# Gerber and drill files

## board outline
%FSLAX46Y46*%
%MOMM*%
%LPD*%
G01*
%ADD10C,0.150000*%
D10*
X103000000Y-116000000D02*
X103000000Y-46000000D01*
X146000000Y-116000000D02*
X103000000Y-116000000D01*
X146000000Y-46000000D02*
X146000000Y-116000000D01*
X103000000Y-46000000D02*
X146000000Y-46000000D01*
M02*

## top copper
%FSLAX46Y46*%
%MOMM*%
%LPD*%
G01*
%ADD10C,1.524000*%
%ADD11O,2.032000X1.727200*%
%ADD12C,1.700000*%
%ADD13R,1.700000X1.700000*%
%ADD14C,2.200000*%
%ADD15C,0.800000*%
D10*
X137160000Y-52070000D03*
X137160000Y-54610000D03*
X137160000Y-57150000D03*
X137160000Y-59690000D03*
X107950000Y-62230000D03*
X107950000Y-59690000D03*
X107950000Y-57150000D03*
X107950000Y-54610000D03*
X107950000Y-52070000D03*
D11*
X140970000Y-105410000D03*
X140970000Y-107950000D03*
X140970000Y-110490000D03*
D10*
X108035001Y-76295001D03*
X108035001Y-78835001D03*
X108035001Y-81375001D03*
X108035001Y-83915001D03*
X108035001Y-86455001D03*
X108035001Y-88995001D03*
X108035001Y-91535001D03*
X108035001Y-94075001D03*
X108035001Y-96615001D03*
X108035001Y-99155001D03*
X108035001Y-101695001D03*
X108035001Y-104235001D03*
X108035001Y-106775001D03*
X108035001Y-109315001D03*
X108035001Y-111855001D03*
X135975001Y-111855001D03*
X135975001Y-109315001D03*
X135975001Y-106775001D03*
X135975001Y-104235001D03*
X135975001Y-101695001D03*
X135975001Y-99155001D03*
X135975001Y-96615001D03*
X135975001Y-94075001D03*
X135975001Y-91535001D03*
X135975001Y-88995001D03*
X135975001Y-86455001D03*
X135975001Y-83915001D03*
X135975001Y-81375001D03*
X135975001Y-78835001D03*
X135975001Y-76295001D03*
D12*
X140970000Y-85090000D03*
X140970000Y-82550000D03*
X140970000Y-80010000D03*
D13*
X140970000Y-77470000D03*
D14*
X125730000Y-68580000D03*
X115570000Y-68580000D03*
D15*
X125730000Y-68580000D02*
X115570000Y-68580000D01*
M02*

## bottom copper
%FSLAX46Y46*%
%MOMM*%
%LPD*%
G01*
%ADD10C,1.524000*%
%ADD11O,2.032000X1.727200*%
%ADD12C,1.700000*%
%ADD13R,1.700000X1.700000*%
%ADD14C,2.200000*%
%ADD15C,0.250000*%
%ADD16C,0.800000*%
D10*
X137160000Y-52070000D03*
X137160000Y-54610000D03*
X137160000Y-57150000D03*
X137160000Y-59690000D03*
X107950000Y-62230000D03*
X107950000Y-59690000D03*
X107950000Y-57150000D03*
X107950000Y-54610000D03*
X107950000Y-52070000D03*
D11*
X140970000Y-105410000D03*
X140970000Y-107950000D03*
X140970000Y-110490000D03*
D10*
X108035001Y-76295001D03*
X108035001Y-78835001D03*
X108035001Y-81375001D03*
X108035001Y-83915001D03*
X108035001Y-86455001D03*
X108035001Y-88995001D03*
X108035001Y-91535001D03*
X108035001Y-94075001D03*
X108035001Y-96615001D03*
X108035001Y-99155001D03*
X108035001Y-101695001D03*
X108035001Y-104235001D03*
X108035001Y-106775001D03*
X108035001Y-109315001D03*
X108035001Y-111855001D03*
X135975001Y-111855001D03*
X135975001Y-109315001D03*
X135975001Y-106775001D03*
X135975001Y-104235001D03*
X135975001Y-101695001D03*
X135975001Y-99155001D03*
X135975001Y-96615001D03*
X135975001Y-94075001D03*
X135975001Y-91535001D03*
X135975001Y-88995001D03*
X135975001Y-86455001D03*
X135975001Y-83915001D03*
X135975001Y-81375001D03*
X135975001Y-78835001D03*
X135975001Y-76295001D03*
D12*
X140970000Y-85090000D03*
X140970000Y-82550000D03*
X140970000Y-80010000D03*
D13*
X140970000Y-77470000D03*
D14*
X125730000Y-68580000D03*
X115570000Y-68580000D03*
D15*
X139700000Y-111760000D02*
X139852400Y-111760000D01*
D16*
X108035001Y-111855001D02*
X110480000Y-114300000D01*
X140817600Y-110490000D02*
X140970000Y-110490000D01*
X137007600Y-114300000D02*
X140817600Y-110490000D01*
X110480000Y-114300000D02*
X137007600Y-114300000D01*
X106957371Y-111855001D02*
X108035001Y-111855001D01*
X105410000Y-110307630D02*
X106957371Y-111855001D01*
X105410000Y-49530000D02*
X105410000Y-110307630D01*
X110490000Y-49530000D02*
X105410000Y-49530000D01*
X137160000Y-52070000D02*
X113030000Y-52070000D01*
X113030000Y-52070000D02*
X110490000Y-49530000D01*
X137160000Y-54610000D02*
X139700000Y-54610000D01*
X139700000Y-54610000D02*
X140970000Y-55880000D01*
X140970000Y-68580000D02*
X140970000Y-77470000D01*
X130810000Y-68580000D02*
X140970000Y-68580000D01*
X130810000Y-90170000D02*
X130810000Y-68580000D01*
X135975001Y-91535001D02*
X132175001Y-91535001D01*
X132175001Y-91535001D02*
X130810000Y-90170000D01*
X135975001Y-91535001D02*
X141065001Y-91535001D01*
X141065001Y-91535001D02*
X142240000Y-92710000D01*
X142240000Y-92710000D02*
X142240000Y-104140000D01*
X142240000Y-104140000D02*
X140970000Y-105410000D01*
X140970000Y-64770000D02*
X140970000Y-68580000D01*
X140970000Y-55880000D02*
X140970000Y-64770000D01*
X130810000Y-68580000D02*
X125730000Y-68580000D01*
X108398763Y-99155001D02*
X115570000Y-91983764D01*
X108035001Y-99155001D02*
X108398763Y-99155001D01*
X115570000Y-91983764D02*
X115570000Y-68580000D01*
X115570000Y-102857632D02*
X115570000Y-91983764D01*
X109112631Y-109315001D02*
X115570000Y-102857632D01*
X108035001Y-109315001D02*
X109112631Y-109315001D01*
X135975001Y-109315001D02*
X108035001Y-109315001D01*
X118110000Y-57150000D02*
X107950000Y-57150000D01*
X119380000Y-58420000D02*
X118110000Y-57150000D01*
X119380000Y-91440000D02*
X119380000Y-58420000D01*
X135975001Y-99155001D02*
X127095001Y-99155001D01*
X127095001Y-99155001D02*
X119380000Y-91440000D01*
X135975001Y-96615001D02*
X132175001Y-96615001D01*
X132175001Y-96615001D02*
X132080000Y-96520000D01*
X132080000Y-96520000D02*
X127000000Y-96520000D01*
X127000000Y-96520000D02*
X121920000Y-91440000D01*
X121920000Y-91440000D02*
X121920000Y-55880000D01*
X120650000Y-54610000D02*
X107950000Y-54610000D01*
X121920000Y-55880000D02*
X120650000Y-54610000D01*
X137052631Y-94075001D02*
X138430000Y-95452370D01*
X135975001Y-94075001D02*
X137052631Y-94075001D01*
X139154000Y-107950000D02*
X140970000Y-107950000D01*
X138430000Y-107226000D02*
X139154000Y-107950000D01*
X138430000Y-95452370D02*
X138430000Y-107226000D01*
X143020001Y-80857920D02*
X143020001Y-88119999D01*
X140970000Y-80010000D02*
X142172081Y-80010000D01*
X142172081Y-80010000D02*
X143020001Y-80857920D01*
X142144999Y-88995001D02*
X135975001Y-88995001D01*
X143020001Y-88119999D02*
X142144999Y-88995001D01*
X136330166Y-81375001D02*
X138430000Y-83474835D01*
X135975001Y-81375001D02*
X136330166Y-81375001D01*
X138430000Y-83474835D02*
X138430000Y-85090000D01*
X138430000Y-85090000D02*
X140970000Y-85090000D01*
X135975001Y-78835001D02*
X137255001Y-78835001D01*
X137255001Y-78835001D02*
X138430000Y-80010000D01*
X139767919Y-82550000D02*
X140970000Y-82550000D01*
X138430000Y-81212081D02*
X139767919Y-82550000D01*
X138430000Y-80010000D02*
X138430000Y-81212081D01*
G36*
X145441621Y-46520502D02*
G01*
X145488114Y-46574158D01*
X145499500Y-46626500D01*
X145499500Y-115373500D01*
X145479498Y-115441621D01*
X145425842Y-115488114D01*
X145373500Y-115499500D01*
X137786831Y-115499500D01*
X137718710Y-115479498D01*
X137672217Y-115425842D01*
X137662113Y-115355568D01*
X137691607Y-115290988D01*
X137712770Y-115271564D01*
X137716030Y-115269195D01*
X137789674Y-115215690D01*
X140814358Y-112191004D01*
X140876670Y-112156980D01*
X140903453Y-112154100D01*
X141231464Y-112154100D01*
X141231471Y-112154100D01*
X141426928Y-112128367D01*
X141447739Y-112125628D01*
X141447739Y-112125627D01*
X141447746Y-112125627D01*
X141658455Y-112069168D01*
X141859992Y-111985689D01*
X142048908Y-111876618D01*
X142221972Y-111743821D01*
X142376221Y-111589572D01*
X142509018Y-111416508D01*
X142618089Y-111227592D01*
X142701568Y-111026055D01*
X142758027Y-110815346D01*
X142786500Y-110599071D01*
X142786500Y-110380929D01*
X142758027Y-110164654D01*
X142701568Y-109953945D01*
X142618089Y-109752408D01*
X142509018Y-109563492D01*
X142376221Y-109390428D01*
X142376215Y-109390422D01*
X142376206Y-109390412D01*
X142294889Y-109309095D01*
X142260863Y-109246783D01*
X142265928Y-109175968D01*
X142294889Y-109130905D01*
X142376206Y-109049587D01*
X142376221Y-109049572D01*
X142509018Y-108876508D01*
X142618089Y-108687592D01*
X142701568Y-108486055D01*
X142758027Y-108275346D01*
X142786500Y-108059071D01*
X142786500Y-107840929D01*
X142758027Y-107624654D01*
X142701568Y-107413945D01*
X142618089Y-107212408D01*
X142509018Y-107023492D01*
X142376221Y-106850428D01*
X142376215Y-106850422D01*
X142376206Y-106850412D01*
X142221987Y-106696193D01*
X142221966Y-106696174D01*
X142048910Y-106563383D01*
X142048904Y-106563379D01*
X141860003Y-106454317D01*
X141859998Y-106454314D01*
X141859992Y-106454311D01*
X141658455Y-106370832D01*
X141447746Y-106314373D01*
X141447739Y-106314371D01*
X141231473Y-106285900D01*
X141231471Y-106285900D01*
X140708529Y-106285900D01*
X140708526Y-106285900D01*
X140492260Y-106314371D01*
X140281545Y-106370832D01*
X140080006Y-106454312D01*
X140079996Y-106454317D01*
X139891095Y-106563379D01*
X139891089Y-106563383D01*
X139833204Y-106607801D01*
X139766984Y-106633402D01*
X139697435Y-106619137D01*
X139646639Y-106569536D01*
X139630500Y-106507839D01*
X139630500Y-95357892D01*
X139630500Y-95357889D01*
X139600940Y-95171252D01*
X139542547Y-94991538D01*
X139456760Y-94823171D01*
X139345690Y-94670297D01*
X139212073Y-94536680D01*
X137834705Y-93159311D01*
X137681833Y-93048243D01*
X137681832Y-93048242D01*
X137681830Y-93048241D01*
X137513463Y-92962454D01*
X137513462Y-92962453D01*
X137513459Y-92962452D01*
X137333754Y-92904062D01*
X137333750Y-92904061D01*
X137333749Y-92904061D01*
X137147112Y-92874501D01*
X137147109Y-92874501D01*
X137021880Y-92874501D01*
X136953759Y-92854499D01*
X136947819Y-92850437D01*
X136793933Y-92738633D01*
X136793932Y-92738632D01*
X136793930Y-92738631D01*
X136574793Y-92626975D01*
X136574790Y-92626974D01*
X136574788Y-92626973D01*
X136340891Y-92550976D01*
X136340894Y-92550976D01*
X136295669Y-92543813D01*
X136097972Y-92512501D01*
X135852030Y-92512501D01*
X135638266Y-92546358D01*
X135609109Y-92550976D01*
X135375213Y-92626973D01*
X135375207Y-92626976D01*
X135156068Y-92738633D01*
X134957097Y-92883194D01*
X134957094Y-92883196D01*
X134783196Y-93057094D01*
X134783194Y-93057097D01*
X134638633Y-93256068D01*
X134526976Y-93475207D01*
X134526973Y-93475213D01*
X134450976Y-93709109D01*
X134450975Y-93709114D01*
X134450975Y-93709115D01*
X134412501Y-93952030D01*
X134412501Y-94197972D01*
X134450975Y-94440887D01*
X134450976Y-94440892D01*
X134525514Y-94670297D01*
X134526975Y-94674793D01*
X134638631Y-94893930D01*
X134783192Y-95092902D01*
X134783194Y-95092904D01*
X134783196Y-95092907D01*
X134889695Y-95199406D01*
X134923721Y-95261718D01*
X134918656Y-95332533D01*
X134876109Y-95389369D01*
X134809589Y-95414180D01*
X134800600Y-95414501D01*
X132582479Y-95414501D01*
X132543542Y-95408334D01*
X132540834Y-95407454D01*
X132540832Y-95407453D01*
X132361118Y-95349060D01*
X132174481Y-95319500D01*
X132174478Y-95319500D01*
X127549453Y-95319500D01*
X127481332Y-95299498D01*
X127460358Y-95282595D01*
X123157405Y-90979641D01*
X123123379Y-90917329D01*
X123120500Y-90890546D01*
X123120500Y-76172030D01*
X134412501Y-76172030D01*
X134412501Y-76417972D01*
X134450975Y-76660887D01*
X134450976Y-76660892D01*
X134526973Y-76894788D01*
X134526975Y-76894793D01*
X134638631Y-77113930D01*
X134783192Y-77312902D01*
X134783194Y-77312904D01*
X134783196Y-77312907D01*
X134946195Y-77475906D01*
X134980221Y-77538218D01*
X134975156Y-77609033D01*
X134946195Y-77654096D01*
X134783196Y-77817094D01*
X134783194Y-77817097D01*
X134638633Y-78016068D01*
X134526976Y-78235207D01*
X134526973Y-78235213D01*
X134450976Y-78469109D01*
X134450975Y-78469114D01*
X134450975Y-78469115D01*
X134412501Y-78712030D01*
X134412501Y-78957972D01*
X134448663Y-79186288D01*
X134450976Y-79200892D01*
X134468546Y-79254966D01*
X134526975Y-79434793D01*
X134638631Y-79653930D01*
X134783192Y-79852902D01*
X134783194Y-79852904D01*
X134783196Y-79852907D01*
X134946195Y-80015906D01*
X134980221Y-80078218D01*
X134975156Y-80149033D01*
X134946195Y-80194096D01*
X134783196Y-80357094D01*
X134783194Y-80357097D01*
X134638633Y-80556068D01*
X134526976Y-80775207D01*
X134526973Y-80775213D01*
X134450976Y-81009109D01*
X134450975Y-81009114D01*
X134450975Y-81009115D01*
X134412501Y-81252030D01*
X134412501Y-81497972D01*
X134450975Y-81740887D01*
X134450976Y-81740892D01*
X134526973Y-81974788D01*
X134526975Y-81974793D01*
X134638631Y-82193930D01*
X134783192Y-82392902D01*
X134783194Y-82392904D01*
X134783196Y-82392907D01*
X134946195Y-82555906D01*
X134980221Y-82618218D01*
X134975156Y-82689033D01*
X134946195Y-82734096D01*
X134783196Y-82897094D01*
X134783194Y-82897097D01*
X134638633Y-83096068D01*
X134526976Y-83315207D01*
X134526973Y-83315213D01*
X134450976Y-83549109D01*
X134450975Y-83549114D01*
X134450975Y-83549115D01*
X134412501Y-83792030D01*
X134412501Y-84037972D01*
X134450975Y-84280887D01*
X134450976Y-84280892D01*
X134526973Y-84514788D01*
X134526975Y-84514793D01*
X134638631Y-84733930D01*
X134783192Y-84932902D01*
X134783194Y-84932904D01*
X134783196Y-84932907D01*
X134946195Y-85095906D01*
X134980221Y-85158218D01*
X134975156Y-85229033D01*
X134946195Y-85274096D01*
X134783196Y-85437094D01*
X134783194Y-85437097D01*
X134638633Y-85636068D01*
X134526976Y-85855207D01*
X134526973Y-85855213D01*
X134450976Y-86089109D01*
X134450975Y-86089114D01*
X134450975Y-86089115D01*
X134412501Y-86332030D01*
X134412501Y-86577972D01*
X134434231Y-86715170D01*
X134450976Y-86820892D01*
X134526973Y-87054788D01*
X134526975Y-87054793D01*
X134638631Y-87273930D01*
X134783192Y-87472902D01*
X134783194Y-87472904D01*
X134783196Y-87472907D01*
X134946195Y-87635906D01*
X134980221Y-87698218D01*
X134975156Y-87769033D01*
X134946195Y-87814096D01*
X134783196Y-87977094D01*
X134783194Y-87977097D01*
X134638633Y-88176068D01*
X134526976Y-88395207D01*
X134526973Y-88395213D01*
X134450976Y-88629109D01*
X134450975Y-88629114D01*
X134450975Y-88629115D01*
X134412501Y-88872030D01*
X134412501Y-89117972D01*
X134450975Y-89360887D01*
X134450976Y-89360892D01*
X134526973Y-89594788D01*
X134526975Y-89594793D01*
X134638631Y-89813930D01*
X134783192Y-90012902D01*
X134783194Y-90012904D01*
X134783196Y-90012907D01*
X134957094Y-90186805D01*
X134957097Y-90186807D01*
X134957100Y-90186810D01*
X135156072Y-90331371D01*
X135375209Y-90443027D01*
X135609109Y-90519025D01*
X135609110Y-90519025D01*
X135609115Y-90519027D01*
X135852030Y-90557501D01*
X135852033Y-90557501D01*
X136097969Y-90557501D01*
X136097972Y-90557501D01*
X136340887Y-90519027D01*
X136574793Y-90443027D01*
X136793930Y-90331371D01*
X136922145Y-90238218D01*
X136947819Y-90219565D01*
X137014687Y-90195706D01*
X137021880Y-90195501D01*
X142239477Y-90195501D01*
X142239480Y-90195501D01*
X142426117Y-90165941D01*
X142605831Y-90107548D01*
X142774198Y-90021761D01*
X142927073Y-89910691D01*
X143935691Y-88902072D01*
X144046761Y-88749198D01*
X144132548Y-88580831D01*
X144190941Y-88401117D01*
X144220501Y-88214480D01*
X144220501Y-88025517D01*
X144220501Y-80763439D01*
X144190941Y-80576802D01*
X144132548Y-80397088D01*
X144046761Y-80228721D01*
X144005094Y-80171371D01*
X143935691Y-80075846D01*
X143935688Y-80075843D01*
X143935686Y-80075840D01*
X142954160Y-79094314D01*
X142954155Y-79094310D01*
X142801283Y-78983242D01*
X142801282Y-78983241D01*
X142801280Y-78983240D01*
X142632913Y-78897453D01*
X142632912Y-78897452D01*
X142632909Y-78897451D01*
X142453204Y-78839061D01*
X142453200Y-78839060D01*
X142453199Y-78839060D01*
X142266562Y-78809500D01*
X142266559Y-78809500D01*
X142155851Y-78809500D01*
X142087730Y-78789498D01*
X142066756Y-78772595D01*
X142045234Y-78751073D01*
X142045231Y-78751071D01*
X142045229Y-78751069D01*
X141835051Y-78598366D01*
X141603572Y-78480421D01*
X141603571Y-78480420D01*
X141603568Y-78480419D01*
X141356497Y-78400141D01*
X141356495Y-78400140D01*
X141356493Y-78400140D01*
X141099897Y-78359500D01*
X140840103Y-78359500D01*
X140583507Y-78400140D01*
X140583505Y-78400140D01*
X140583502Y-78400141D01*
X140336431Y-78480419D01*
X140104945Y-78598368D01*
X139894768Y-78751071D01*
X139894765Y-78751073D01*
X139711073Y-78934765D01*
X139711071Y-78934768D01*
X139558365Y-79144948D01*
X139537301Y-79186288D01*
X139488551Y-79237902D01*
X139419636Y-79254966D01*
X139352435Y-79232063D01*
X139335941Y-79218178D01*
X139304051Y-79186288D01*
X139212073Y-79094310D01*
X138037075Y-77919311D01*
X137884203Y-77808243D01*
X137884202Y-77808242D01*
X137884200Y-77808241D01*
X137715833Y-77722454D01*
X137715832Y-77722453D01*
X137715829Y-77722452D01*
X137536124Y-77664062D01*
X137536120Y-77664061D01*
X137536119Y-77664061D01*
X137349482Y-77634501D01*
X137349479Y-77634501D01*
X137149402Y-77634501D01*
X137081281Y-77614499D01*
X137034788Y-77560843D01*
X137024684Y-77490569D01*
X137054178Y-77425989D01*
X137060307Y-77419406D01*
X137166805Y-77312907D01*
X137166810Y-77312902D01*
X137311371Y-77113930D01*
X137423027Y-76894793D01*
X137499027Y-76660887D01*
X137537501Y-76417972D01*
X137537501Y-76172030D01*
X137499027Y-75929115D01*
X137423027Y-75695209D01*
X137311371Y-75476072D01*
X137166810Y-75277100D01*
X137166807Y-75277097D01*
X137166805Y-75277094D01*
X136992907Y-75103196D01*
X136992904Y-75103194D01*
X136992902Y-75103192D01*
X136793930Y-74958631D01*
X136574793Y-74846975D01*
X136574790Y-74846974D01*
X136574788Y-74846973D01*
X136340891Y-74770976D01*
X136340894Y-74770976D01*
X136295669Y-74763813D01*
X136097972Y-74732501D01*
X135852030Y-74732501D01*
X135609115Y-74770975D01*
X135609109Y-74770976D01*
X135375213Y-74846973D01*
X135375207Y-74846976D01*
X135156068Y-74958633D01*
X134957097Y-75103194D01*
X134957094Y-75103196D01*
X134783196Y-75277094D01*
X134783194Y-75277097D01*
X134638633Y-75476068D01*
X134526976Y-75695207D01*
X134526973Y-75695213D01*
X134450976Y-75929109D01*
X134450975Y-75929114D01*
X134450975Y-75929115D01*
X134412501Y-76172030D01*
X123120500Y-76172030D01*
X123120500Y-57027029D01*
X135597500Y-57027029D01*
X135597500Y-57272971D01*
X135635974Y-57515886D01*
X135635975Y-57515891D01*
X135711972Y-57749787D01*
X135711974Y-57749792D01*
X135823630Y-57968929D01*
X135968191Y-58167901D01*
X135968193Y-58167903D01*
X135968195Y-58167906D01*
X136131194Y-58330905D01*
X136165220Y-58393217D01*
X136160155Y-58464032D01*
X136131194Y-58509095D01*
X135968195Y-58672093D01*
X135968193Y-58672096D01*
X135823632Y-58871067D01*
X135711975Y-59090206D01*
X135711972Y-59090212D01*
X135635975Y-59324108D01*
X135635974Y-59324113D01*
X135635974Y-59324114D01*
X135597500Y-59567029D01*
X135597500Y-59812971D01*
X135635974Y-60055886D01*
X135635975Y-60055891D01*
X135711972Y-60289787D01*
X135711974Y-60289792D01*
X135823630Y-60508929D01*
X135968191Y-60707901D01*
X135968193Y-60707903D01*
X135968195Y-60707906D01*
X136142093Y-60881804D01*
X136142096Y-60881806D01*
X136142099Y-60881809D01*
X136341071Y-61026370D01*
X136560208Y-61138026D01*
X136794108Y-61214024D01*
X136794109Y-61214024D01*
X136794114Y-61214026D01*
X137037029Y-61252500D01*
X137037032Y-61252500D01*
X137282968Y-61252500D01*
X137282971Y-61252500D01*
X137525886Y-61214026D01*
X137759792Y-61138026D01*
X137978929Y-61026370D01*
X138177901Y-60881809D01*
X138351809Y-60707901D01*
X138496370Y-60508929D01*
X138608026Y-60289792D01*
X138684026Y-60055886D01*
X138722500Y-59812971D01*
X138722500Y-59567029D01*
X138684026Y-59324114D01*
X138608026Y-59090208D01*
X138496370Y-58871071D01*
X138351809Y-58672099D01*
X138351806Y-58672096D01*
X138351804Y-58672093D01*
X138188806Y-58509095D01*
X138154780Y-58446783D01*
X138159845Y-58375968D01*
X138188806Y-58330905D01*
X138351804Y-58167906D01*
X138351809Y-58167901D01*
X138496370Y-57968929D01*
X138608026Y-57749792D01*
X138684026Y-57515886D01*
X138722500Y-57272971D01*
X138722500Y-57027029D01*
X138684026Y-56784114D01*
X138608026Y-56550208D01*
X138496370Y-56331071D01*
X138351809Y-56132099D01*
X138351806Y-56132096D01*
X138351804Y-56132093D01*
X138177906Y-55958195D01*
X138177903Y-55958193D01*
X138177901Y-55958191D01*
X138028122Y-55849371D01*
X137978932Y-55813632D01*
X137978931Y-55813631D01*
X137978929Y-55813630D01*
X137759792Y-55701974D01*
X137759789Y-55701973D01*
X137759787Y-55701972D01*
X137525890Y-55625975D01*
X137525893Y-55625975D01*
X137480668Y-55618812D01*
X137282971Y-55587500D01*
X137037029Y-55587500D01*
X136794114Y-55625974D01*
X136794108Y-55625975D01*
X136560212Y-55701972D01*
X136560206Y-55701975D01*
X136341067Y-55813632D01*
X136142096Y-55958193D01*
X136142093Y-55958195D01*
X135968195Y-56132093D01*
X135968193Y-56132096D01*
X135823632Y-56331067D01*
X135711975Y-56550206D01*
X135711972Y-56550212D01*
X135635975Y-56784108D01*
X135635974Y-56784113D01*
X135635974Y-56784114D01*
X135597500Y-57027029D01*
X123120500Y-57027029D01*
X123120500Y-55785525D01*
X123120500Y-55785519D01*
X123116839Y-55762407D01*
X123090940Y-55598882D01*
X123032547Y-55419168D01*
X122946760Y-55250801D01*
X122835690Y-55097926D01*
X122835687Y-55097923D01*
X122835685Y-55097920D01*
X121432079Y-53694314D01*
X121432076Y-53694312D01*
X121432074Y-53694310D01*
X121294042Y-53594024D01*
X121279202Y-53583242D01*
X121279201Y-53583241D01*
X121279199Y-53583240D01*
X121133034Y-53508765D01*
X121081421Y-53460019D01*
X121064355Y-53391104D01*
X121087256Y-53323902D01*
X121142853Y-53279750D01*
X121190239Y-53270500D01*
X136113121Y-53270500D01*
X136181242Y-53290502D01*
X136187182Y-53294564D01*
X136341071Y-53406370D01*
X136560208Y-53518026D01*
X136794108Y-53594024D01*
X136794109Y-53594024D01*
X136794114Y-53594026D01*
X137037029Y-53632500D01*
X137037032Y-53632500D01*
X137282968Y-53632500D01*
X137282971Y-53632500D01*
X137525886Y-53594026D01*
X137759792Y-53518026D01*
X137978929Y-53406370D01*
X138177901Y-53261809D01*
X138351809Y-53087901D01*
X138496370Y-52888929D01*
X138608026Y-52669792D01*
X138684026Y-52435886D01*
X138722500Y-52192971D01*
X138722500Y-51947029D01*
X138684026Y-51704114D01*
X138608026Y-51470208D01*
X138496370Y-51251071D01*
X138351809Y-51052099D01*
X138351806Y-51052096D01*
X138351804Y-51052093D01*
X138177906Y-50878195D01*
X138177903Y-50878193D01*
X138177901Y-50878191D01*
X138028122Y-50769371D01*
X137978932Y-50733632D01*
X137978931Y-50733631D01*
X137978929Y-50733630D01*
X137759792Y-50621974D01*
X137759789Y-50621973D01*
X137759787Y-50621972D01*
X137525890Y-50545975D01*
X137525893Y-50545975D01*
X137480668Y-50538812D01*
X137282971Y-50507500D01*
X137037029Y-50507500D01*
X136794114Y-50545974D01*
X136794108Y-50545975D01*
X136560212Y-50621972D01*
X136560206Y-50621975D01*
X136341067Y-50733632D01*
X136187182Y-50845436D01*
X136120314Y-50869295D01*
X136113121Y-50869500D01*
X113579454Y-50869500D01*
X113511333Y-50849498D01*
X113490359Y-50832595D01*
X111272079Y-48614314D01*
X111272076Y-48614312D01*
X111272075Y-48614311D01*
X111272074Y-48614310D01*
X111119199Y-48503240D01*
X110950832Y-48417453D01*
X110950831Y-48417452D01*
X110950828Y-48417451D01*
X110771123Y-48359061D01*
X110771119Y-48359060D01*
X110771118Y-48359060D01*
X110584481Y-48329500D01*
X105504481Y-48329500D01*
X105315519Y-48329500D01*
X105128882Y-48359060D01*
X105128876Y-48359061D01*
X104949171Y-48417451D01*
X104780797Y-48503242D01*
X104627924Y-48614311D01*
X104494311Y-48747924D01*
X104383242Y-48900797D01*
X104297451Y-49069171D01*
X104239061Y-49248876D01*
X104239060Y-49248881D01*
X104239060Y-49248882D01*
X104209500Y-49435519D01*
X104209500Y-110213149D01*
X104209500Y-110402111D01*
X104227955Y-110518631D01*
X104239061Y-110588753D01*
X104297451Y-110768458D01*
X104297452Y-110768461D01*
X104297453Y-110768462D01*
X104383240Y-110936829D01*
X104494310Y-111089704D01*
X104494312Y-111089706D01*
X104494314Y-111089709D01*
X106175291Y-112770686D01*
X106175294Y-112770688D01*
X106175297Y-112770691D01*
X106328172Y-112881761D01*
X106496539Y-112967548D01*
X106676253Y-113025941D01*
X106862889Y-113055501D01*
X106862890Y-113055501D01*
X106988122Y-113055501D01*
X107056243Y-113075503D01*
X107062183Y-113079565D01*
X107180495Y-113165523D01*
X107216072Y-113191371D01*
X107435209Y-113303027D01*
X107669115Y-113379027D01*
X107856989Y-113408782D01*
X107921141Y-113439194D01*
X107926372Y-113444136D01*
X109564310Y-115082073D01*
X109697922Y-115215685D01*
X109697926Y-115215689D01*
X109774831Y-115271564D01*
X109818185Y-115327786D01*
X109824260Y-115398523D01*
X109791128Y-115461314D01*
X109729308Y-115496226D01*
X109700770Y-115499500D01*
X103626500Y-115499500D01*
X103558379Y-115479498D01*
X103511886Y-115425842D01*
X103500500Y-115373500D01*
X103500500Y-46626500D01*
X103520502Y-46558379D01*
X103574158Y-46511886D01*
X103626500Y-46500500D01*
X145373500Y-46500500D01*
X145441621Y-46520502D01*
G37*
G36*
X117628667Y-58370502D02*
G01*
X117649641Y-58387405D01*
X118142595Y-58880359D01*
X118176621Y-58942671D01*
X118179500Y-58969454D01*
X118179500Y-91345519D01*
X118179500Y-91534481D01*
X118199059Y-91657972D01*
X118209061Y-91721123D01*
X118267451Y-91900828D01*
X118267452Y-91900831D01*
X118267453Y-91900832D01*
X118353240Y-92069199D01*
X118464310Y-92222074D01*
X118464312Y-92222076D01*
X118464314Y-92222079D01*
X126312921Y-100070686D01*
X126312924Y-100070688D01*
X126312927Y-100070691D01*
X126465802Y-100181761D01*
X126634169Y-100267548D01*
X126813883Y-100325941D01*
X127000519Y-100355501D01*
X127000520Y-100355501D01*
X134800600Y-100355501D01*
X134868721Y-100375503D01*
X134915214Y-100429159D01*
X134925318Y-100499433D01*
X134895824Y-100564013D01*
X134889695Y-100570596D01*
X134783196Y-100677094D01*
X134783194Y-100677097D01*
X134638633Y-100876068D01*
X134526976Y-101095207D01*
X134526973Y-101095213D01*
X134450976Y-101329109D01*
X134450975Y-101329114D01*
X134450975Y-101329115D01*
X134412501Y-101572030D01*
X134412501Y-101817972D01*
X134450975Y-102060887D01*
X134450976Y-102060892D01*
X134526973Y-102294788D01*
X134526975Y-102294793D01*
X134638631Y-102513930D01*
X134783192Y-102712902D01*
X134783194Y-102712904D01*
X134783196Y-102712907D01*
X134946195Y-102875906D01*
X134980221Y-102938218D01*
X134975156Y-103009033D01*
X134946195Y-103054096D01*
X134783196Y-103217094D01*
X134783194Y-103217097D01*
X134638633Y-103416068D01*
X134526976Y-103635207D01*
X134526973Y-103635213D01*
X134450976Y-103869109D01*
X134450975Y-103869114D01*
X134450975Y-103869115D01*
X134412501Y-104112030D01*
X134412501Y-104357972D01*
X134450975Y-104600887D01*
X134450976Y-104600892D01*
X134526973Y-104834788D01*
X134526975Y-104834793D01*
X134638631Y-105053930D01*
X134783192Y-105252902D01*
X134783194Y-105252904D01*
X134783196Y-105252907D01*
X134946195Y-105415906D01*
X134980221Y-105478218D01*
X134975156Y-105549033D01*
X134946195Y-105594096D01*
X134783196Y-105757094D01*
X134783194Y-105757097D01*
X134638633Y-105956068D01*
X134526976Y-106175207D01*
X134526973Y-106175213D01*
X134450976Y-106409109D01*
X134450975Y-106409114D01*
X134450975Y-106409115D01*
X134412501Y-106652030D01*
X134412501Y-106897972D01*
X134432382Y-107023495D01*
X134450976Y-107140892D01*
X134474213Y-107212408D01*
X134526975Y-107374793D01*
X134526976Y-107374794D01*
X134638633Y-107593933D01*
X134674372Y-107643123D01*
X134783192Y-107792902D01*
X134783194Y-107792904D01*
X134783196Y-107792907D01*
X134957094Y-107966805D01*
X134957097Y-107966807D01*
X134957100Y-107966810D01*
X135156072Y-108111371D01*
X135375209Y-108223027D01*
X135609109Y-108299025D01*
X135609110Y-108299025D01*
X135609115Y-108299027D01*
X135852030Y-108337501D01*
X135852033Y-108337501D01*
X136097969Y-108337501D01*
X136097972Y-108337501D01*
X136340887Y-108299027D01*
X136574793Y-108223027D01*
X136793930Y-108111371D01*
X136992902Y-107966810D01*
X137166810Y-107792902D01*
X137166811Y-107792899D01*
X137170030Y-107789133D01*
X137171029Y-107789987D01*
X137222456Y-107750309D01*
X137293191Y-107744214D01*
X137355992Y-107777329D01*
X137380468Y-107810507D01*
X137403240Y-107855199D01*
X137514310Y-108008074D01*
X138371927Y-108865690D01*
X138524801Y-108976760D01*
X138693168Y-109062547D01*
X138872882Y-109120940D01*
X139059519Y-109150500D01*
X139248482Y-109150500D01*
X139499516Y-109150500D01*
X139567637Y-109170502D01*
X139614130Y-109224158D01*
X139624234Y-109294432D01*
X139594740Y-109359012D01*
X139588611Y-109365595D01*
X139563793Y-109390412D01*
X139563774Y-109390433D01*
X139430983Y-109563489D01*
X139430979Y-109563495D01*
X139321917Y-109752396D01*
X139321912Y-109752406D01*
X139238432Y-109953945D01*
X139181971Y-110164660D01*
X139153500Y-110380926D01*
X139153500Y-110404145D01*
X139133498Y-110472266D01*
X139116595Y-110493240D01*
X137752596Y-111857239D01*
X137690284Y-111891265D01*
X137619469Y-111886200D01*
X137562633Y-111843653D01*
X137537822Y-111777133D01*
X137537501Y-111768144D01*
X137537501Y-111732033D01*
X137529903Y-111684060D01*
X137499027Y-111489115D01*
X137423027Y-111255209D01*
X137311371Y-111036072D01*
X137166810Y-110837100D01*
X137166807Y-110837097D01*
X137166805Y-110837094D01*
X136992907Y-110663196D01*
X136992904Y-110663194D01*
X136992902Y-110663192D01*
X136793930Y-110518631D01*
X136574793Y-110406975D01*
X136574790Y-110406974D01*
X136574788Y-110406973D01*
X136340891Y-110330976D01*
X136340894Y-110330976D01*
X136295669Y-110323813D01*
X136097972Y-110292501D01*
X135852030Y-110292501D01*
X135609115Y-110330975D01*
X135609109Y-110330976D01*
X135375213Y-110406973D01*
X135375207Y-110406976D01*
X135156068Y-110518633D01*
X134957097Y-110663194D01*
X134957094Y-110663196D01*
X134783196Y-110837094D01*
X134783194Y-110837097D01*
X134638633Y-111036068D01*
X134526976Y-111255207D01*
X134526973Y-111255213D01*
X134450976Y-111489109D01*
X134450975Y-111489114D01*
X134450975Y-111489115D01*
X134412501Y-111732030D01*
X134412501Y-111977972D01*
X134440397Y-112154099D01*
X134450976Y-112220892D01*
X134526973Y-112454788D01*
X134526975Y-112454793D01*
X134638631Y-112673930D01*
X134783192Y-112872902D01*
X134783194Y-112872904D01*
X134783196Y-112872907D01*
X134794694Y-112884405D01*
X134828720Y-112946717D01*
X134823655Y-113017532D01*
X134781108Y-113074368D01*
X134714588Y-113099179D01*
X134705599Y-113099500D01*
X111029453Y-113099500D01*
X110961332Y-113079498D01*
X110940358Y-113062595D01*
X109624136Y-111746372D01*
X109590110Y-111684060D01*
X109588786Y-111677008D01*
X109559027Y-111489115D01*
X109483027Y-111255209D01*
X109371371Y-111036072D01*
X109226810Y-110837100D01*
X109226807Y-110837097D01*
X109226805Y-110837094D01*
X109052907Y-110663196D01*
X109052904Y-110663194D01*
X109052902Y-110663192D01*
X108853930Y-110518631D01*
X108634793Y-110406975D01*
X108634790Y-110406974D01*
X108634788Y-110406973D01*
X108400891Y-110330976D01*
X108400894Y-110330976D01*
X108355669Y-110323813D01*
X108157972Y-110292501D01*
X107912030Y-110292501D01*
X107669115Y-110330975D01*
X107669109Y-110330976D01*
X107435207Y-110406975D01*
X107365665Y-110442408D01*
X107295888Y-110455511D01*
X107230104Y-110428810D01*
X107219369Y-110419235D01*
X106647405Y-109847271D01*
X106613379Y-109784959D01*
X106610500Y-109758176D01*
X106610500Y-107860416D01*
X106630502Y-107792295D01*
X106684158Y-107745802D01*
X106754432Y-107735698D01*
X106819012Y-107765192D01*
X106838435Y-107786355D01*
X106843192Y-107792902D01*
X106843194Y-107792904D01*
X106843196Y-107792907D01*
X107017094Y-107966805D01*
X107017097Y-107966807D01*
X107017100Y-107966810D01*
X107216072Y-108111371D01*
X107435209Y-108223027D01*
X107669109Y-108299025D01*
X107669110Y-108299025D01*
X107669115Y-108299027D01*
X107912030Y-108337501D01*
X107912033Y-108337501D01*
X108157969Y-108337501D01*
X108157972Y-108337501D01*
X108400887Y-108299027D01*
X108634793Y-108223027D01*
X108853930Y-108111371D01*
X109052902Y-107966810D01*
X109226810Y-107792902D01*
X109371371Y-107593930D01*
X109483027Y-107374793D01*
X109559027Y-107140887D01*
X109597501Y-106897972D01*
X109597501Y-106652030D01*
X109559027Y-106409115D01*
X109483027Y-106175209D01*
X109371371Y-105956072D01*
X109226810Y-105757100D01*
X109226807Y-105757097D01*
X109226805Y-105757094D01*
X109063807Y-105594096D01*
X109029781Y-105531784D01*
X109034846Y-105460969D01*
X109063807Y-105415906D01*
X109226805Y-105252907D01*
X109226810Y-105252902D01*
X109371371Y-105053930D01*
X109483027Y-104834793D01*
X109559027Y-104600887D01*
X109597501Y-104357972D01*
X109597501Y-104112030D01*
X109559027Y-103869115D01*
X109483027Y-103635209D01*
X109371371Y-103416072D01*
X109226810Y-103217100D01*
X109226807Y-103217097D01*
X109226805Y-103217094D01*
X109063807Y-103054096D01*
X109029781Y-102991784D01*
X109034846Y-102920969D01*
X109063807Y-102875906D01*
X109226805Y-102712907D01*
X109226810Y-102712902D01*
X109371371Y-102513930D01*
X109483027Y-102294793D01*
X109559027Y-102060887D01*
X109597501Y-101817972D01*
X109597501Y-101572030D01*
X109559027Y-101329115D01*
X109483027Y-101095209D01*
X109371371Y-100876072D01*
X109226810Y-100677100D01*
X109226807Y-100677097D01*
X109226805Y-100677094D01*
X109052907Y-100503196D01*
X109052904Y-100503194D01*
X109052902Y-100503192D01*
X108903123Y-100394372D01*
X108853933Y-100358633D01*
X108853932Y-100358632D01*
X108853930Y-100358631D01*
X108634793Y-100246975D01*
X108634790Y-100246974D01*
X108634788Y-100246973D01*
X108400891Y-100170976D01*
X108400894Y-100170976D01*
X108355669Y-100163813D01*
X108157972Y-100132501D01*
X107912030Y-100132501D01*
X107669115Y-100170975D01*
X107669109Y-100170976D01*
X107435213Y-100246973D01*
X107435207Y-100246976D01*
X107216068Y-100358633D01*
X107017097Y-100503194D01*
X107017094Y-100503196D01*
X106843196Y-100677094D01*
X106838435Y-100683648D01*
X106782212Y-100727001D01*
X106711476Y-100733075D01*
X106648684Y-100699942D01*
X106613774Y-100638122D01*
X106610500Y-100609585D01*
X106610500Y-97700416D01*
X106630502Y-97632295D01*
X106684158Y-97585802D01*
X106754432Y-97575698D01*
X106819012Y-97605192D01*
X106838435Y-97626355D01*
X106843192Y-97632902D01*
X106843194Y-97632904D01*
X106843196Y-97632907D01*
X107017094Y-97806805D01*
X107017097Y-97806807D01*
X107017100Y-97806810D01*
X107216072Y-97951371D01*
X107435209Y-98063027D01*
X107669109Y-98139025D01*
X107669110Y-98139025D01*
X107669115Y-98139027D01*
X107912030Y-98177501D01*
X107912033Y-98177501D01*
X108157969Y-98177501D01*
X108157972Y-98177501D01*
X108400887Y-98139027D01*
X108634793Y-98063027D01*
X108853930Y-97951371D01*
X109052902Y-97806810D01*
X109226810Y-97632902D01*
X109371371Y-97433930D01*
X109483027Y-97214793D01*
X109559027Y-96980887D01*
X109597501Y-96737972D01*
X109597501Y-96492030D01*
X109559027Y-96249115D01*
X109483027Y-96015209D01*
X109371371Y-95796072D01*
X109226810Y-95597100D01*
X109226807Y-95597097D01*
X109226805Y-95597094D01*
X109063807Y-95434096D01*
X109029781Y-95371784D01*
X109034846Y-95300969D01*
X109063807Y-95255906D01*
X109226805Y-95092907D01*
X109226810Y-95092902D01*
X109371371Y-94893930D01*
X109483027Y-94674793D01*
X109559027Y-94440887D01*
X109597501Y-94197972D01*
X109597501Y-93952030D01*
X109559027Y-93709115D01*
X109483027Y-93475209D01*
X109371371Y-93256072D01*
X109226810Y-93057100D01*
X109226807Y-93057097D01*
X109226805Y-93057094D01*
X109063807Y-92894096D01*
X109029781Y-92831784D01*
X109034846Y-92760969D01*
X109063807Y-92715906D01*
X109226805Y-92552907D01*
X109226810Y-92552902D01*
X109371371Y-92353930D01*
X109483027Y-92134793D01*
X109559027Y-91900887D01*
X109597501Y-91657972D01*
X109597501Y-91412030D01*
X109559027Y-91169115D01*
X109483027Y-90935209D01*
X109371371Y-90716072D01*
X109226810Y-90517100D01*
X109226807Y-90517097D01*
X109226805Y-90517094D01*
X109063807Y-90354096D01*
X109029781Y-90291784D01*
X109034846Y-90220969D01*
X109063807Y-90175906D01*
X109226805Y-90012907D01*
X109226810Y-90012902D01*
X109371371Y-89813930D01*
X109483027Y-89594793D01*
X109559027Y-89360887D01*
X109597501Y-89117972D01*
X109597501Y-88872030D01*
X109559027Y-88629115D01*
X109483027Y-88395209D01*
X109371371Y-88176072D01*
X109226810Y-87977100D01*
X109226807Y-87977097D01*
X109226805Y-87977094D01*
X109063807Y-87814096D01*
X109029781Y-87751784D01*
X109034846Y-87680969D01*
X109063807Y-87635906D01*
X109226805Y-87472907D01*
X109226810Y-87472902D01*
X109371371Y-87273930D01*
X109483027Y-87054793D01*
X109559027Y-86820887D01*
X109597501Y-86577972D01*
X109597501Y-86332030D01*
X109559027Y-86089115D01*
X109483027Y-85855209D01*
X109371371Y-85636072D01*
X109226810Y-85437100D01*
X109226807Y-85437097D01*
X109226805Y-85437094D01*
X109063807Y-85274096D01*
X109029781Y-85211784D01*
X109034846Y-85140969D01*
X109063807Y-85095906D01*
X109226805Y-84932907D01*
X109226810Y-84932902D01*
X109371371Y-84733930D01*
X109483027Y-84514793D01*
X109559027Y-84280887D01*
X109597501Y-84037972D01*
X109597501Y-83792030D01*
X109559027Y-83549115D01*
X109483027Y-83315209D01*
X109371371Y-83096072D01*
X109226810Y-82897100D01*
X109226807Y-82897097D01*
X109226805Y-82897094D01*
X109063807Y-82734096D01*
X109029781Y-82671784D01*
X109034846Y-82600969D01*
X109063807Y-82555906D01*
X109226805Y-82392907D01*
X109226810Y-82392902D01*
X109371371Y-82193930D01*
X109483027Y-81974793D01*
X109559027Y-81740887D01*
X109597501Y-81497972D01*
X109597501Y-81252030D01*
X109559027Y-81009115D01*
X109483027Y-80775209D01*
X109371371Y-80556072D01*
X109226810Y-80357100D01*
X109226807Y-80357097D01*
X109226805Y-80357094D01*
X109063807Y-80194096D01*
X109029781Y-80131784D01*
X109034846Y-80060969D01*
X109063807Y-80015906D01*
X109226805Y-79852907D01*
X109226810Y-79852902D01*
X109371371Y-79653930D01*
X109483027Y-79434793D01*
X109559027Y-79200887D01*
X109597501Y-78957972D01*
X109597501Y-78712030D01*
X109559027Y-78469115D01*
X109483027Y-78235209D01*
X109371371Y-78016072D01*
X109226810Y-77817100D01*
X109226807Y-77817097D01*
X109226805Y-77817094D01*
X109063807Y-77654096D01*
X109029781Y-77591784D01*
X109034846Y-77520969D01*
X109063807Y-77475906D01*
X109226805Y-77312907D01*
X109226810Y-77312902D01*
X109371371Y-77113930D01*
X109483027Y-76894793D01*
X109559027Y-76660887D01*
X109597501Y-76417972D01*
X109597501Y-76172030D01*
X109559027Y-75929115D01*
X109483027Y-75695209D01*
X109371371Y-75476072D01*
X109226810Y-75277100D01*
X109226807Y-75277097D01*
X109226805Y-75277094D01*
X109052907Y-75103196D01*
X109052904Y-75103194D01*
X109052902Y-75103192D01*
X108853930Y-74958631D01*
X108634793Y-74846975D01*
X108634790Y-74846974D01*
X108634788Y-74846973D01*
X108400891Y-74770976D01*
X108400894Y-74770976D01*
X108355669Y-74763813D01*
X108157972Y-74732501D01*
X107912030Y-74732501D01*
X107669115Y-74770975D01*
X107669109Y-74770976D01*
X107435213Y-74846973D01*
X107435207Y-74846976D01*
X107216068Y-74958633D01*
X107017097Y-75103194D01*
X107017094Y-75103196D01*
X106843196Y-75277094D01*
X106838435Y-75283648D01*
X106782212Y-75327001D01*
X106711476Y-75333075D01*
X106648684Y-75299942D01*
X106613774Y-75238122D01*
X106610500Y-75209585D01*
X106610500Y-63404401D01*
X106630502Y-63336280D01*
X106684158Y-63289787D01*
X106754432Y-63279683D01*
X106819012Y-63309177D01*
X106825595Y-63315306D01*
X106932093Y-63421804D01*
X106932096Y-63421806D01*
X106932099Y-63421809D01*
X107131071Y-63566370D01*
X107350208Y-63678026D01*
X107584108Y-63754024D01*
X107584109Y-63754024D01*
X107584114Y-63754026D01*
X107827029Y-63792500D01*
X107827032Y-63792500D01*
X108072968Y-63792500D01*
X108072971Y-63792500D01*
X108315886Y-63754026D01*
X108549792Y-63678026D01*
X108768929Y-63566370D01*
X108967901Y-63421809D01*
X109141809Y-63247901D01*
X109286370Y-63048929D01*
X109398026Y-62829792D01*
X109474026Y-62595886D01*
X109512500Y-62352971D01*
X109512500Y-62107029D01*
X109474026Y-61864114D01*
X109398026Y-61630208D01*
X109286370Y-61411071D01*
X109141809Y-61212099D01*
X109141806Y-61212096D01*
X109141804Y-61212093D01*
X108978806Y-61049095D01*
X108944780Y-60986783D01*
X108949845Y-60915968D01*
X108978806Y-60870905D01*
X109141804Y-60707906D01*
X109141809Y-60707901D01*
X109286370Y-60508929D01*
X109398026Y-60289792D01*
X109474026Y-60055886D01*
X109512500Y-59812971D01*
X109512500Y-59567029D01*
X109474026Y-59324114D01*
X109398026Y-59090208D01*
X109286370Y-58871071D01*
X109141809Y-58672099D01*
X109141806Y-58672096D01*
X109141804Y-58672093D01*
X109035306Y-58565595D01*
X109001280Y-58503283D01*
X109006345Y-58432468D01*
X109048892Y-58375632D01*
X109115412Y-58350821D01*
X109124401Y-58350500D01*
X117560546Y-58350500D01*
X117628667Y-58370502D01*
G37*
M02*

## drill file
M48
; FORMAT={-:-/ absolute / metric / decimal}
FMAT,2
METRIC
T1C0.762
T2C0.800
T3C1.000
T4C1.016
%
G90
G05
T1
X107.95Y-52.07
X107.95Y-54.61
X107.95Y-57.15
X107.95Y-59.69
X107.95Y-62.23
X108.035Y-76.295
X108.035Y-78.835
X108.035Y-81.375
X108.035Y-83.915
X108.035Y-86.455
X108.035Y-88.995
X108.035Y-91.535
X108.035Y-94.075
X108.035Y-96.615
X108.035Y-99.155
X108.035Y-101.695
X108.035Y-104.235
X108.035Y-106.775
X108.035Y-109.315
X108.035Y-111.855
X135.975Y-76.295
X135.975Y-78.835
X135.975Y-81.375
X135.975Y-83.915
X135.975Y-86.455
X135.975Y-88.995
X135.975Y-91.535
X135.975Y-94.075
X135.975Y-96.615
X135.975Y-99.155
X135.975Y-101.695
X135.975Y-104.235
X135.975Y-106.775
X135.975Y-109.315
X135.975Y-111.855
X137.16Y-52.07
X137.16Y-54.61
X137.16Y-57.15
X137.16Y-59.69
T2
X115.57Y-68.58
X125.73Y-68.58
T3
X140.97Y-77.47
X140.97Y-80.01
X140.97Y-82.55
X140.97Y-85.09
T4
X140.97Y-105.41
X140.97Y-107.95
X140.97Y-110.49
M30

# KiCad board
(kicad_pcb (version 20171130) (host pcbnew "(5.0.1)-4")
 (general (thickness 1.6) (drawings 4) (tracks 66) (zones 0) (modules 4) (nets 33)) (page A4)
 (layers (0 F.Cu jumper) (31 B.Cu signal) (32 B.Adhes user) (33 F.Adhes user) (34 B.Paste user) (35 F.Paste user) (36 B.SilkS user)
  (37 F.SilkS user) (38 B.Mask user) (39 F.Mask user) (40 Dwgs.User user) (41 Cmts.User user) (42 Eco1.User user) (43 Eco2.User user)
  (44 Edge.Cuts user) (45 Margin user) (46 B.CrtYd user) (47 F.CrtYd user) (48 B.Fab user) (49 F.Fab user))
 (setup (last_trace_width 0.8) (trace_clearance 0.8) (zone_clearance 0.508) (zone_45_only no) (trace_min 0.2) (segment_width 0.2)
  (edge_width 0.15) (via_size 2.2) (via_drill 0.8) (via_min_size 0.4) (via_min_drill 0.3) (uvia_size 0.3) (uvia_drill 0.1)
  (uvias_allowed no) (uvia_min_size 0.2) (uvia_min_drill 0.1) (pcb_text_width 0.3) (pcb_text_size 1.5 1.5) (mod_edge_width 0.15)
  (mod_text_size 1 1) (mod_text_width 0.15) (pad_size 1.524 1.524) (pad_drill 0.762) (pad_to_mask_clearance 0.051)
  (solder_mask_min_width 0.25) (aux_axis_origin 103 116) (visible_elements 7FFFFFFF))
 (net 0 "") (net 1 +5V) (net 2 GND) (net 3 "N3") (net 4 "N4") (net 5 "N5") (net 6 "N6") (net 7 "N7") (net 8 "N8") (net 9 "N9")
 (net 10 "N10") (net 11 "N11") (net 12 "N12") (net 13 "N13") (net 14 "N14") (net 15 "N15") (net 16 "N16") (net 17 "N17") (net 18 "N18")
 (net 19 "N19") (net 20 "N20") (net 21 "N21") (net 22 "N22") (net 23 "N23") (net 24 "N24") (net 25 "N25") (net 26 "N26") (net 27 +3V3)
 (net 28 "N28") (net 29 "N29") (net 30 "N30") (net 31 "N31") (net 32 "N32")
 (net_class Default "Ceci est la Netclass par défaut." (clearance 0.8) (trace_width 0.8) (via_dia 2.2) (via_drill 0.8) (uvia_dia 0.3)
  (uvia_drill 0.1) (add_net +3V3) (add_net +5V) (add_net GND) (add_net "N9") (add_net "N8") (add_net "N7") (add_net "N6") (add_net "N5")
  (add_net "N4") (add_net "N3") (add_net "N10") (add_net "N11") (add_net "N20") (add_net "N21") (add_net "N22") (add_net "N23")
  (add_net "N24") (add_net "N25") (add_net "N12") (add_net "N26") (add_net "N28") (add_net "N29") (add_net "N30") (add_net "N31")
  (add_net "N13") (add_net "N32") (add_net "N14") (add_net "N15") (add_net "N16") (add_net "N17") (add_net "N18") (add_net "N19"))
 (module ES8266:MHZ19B (layer F.Cu) (at 107.95 52.07)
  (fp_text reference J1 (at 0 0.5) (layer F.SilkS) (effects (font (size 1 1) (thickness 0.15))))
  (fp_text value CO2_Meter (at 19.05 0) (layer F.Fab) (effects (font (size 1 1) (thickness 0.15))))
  (pad 9 thru_hole circle (at 29.21 0) (size 1.524 1.524) (drill 0.762) (layers *.Cu *.Mask) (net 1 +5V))
  (pad 8 thru_hole circle (at 29.21 2.54) (size 1.524 1.524) (drill 0.762) (layers *.Cu *.Mask) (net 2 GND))
  (pad 7 thru_hole circle (at 29.21 5.08) (size 1.524 1.524) (drill 0.762) (layers *.Cu *.Mask) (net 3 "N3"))
  (pad 6 thru_hole circle (at 29.21 7.62) (size 1.524 1.524) (drill 0.762) (layers *.Cu *.Mask) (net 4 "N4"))
  (pad 5 thru_hole circle (at 0 10.16) (size 1.524 1.524) (drill 0.762) (layers *.Cu *.Mask) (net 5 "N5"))
  (pad 4 thru_hole circle (at 0 7.62) (size 1.524 1.524) (drill 0.762) (layers *.Cu *.Mask) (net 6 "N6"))
  (pad 3 thru_hole circle (at 0 5.08) (size 1.524 1.524) (drill 0.762) (layers *.Cu *.Mask) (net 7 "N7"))
  (pad 2 thru_hole circle (at 0 2.54) (size 1.524 1.524) (drill 0.762) (layers *.Cu *.Mask) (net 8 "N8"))
  (pad 1 thru_hole circle (at 0 0) (size 1.524 1.524) (drill 0.762) (layers *.Cu *.Mask) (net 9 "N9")))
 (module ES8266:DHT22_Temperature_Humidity (layer F.Cu) (at 140.97 107.95 90)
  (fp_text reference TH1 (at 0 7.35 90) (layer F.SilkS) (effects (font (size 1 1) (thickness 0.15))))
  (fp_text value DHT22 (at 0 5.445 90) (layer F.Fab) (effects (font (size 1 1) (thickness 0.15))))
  (pad 3 thru_hole oval (at 2.54 0 180) (size 2.032 1.7272) (drill 1.016) (layers *.Cu *.Mask F.SilkS) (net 2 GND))
  (pad 2 thru_hole oval (at 0 0 180) (size 2.032 1.7272) (drill 1.016) (layers *.Cu *.Mask F.SilkS) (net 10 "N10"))
  (pad 1 thru_hole oval (at -2.54 0 180) (size 2.032 1.7272) (drill 1.016) (layers *.Cu *.Mask F.SilkS) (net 1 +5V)))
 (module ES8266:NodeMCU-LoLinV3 (layer F.Cu) (at 122.005001 96.615001)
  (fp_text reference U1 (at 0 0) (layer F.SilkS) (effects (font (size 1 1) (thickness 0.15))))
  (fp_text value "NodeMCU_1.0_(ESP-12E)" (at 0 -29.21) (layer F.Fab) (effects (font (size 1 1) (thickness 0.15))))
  (pad 1 thru_hole circle (at -13.97 -20.32) (size 1.524 1.524) (drill 0.762) (layers *.Cu *.Mask F.SilkS) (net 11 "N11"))
  (pad 2 thru_hole circle (at -13.97 -17.78) (size 1.524 1.524) (drill 0.762) (layers *.Cu *.Mask F.SilkS) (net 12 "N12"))
  (pad 3 thru_hole circle (at -13.97 -15.24) (size 1.524 1.524) (drill 0.762) (layers *.Cu *.Mask F.SilkS) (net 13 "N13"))
  (pad 4 thru_hole circle (at -13.97 -12.7) (size 1.524 1.524) (drill 0.762) (layers *.Cu *.Mask F.SilkS) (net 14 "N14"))
  (pad 5 thru_hole circle (at -13.97 -10.16) (size 1.524 1.524) (drill 0.762) (layers *.Cu *.Mask F.SilkS) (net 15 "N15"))
  (pad 6 thru_hole circle (at -13.97 -7.62) (size 1.524 1.524) (drill 0.762) (layers *.Cu *.Mask F.SilkS) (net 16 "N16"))
  (pad 7 thru_hole circle (at -13.97 -5.08) (size 1.524 1.524) (drill 0.762) (layers *.Cu *.Mask F.SilkS) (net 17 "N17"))
  (pad 8 thru_hole circle (at -13.97 -2.54) (size 1.524 1.524) (drill 0.762) (layers *.Cu *.Mask F.SilkS) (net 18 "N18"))
  (pad 9 thru_hole circle (at -13.97 0) (size 1.524 1.524) (drill 0.762) (layers *.Cu *.Mask F.SilkS) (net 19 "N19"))
  (pad 10 thru_hole circle (at -13.97 2.54) (size 1.524 1.524) (drill 0.762) (layers *.Cu *.Mask F.SilkS) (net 2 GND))
  (pad 11 thru_hole circle (at -13.97 5.08) (size 1.524 1.524) (drill 0.762) (layers *.Cu *.Mask F.SilkS) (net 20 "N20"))
  (pad 12 thru_hole circle (at -13.97 7.62) (size 1.524 1.524) (drill 0.762) (layers *.Cu *.Mask F.SilkS) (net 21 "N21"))
  (pad 13 thru_hole circle (at -13.97 10.16) (size 1.524 1.524) (drill 0.762) (layers *.Cu *.Mask F.SilkS) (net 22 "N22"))
  (pad 14 thru_hole circle (at -13.97 12.7) (size 1.524 1.524) (drill 0.762) (layers *.Cu *.Mask F.SilkS) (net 2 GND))
  (pad 15 thru_hole circle (at -13.97 15.24) (size 1.524 1.524) (drill 0.762) (layers *.Cu *.Mask F.SilkS) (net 1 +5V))
  (pad 16 thru_hole circle (at 13.97 15.24) (size 1.524 1.524) (drill 0.762) (layers *.Cu *.Mask F.SilkS) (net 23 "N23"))
  (pad 17 thru_hole circle (at 13.97 12.7) (size 1.524 1.524) (drill 0.762) (layers *.Cu *.Mask F.SilkS) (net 2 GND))
  (pad 18 thru_hole circle (at 13.97 10.16) (size 1.524 1.524) (drill 0.762) (layers *.Cu *.Mask F.SilkS) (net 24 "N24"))
  (pad 19 thru_hole circle (at 13.97 7.62) (size 1.524 1.524) (drill 0.762) (layers *.Cu *.Mask F.SilkS) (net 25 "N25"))
  (pad 20 thru_hole circle (at 13.97 5.08) (size 1.524 1.524) (drill 0.762) (layers *.Cu *.Mask F.SilkS) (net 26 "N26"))
  (pad 21 thru_hole circle (at 13.97 2.54) (size 1.524 1.524) (drill 0.762) (layers *.Cu *.Mask F.SilkS) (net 7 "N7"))
  (pad 22 thru_hole circle (at 13.97 0) (size 1.524 1.524) (drill 0.762) (layers *.Cu *.Mask F.SilkS) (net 8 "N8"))
  (pad 23 thru_hole circle (at 13.97 -2.54) (size 1.524 1.524) (drill 0.762) (layers *.Cu *.Mask F.SilkS) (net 10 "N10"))
  (pad 24 thru_hole circle (at 13.97 -5.08) (size 1.524 1.524) (drill 0.762) (layers *.Cu *.Mask F.SilkS) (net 2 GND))
  (pad 25 thru_hole circle (at 13.97 -7.62) (size 1.524 1.524) (drill 0.762) (layers *.Cu *.Mask F.SilkS) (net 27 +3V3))
  (pad 26 thru_hole circle (at 13.97 -10.16) (size 1.524 1.524) (drill 0.762) (layers *.Cu *.Mask F.SilkS) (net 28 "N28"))
  (pad 27 thru_hole circle (at 13.97 -12.7) (size 1.524 1.524) (drill 0.762) (layers *.Cu *.Mask F.SilkS) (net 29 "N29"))
  (pad 28 thru_hole circle (at 13.97 -15.24) (size 1.524 1.524) (drill 0.762) (layers *.Cu *.Mask F.SilkS) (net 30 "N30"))
  (pad 29 thru_hole circle (at 13.97 -17.78) (size 1.524 1.524) (drill 0.762) (layers *.Cu *.Mask F.SilkS) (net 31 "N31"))
  (pad 30 thru_hole circle (at 13.97 -20.32) (size 1.524 1.524) (drill 0.762) (layers *.Cu *.Mask F.SilkS) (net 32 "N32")))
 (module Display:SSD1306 (layer F.Cu) (at 140.97 72.39 270)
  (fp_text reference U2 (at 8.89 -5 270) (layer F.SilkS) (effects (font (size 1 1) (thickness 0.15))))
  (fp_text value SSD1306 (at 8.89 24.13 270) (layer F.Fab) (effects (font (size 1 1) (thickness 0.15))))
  (pad 4 thru_hole circle (at 12.7 0 270) (size 1.7 1.7) (drill 1) (layers *.Cu *.Mask) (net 30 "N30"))
  (pad 3 thru_hole circle (at 10.16 0 270) (size 1.7 1.7) (drill 1) (layers *.Cu *.Mask) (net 31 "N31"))
  (pad 2 thru_hole circle (at 7.62 0 270) (size 1.7 1.7) (drill 1) (layers *.Cu *.Mask) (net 27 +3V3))
  (pad 1 thru_hole rect (at 5.08 0 270) (size 1.7 1.7) (drill 1) (layers *.Cu *.Mask) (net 2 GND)))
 (gr_line (start 103 116) (end 103 46) (layer Edge.Cuts) (width 0.15))
 (gr_line (start 146 116) (end 103 116) (layer Edge.Cuts) (width 0.15))
 (gr_line (start 146 46) (end 146 116) (layer Edge.Cuts) (width 0.15))
 (gr_line (start 103 46) (end 146 46) (layer Edge.Cuts) (width 0.15))
 (segment (start 139.7 111.76) (end 139.8524 111.76) (width 0.25) (layer B.Cu) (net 1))
 (segment (start 108.035001 111.855001) (end 110.48 114.3) (width 0.8) (layer B.Cu) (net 1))
 (segment (start 140.8176 110.49) (end 140.97 110.49) (width 0.8) (layer B.Cu) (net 1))
 (segment (start 137.0076 114.3) (end 140.8176 110.49) (width 0.8) (layer B.Cu) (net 1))
 (segment (start 110.48 114.3) (end 137.0076 114.3) (width 0.8) (layer B.Cu) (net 1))
 (segment (start 106.957371 111.855001) (end 108.035001 111.855001) (width 0.8) (layer B.Cu) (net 1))
 (segment (start 105.41 110.30763) (end 106.957371 111.855001) (width 0.8) (layer B.Cu) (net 1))
 (segment (start 105.41 49.53) (end 105.41 110.30763) (width 0.8) (layer B.Cu) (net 1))
 (segment (start 110.49 49.53) (end 105.41 49.53) (width 0.8) (layer B.Cu) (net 1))
 (segment (start 137.16 52.07) (end 113.03 52.07) (width 0.8) (layer B.Cu) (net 1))
 (segment (start 113.03 52.07) (end 110.49 49.53) (width 0.8) (layer B.Cu) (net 1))
 (segment (start 137.16 54.61) (end 139.7 54.61) (width 0.8) (layer B.Cu) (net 2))
 (segment (start 139.7 54.61) (end 140.97 55.88) (width 0.8) (layer B.Cu) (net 2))
 (segment (start 140.97 68.58) (end 140.97 77.47) (width 0.8) (layer B.Cu) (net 2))
 (segment (start 130.81 68.58) (end 140.97 68.58) (width 0.8) (layer B.Cu) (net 2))
 (segment (start 130.81 90.17) (end 130.81 68.58) (width 0.8) (layer B.Cu) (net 2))
 (segment (start 135.975001 91.535001) (end 132.175001 91.535001) (width 0.8) (layer B.Cu) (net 2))
 (segment (start 132.175001 91.535001) (end 130.81 90.17) (width 0.8) (layer B.Cu) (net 2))
 (segment (start 135.975001 91.535001) (end 141.065001 91.535001) (width 0.8) (layer B.Cu) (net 2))
 (segment (start 141.065001 91.535001) (end 142.24 92.71) (width 0.8) (layer B.Cu) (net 2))
 (segment (start 142.24 92.71) (end 142.24 104.14) (width 0.8) (layer B.Cu) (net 2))
 (segment (start 142.24 104.14) (end 140.97 105.41) (width 0.8) (layer B.Cu) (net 2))
 (segment (start 140.97 64.77) (end 140.97 68.58) (width 0.8) (layer B.Cu) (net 2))
 (segment (start 140.97 55.88) (end 140.97 64.77) (width 0.8) (layer B.Cu) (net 2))
 (segment (start 130.81 68.58) (end 125.73 68.58) (width 0.8) (layer B.Cu) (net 2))
 (via (at 125.73 68.58) (size 2.2) (drill 0.8) (layers F.Cu B.Cu) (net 2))
 (segment (start 108.398763 99.155001) (end 115.57 91.983764) (width 0.8) (layer B.Cu) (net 2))
 (segment (start 108.035001 99.155001) (end 108.398763 99.155001) (width 0.8) (layer B.Cu) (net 2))
 (segment (start 115.57 91.983764) (end 115.57 68.58) (width 0.8) (layer B.Cu) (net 2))
 (via (at 115.57 68.58) (size 2.2) (drill 0.8) (layers F.Cu B.Cu) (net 2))
 (segment (start 115.57 102.857632) (end 115.57 91.983764) (width 0.8) (layer B.Cu) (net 2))
 (segment (start 109.112631 109.315001) (end 115.57 102.857632) (width 0.8) (layer B.Cu) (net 2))
 (segment (start 108.035001 109.315001) (end 109.112631 109.315001) (width 0.8) (layer B.Cu) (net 2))
 (segment (start 135.975001 109.315001) (end 108.035001 109.315001) (width 0.8) (layer B.Cu) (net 2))
 (segment (start 125.73 68.58) (end 115.57 68.58) (width 0.8) (layer F.Cu) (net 2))
 (segment (start 118.11 57.15) (end 107.95 57.15) (width 0.8) (layer B.Cu) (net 7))
 (segment (start 119.38 58.42) (end 118.11 57.15) (width 0.8) (layer B.Cu) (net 7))
 (segment (start 119.38 91.44) (end 119.38 58.42) (width 0.8) (layer B.Cu) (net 7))
 (segment (start 135.975001 99.155001) (end 127.095001 99.155001) (width 0.8) (layer B.Cu) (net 7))
 (segment (start 127.095001 99.155001) (end 119.38 91.44) (width 0.8) (layer B.Cu) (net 7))
 (segment (start 135.975001 96.615001) (end 132.175001 96.615001) (width 0.8) (layer B.Cu) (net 8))
 (segment (start 132.175001 96.615001) (end 132.08 96.52) (width 0.8) (layer B.Cu) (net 8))
 (segment (start 132.08 96.52) (end 127 96.52) (width 0.8) (layer B.Cu) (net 8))
 (segment (start 127 96.52) (end 121.92 91.44) (width 0.8) (layer B.Cu) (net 8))
 (segment (start 121.92 91.44) (end 121.92 55.88) (width 0.8) (layer B.Cu) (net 8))
 (segment (start 120.65 54.61) (end 107.95 54.61) (width 0.8) (layer B.Cu) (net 8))
 (segment (start 121.92 55.88) (end 120.65 54.61) (width 0.8) (layer B.Cu) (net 8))
 (segment (start 137.052631 94.075001) (end 138.43 95.45237) (width 0.8) (layer B.Cu) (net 10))
 (segment (start 135.975001 94.075001) (end 137.052631 94.075001) (width 0.8) (layer B.Cu) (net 10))
 (segment (start 139.154 107.95) (end 140.97 107.95) (width 0.8) (layer B.Cu) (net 10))
 (segment (start 138.43 107.226) (end 139.154 107.95) (width 0.8) (layer B.Cu) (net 10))
 (segment (start 138.43 95.45237) (end 138.43 107.226) (width 0.8) (layer B.Cu) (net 10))
 (segment (start 143.020001 80.85792) (end 143.020001 88.119999) (width 0.8) (layer B.Cu) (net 27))
 (segment (start 140.97 80.01) (end 142.172081 80.01) (width 0.8) (layer B.Cu) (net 27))
 (segment (start 142.172081 80.01) (end 143.020001 80.85792) (width 0.8) (layer B.Cu) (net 27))
 (segment (start 142.144999 88.995001) (end 135.975001 88.995001) (width 0.8) (layer B.Cu) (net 27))
 (segment (start 143.020001 88.119999) (end 142.144999 88.995001) (width 0.8) (layer B.Cu) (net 27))
 (segment (start 136.330166 81.375001) (end 138.43 83.474835) (width 0.8) (layer B.Cu) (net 30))
 (segment (start 135.975001 81.375001) (end 136.330166 81.375001) (width 0.8) (layer B.Cu) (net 30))
 (segment (start 138.43 83.474835) (end 138.43 85.09) (width 0.8) (layer B.Cu) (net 30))
 (segment (start 138.43 85.09) (end 140.97 85.09) (width 0.8) (layer B.Cu) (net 30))
 (segment (start 135.975001 78.835001) (end 137.255001 78.835001) (width 0.8) (layer B.Cu) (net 31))
 (segment (start 137.255001 78.835001) (end 138.43 80.01) (width 0.8) (layer B.Cu) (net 31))
 (segment (start 139.767919 82.55) (end 140.97 82.55) (width 0.8) (layer B.Cu) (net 31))
 (segment (start 138.43 81.212081) (end 139.767919 82.55) (width 0.8) (layer B.Cu) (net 31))
 (segment (start 138.43 80.01) (end 138.43 81.212081) (width 0.8) (layer B.Cu) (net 31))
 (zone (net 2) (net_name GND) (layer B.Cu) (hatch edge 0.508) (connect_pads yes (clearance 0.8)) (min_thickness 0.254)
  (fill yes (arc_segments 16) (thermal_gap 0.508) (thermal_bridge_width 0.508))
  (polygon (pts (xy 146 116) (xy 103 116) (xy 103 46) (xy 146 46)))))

